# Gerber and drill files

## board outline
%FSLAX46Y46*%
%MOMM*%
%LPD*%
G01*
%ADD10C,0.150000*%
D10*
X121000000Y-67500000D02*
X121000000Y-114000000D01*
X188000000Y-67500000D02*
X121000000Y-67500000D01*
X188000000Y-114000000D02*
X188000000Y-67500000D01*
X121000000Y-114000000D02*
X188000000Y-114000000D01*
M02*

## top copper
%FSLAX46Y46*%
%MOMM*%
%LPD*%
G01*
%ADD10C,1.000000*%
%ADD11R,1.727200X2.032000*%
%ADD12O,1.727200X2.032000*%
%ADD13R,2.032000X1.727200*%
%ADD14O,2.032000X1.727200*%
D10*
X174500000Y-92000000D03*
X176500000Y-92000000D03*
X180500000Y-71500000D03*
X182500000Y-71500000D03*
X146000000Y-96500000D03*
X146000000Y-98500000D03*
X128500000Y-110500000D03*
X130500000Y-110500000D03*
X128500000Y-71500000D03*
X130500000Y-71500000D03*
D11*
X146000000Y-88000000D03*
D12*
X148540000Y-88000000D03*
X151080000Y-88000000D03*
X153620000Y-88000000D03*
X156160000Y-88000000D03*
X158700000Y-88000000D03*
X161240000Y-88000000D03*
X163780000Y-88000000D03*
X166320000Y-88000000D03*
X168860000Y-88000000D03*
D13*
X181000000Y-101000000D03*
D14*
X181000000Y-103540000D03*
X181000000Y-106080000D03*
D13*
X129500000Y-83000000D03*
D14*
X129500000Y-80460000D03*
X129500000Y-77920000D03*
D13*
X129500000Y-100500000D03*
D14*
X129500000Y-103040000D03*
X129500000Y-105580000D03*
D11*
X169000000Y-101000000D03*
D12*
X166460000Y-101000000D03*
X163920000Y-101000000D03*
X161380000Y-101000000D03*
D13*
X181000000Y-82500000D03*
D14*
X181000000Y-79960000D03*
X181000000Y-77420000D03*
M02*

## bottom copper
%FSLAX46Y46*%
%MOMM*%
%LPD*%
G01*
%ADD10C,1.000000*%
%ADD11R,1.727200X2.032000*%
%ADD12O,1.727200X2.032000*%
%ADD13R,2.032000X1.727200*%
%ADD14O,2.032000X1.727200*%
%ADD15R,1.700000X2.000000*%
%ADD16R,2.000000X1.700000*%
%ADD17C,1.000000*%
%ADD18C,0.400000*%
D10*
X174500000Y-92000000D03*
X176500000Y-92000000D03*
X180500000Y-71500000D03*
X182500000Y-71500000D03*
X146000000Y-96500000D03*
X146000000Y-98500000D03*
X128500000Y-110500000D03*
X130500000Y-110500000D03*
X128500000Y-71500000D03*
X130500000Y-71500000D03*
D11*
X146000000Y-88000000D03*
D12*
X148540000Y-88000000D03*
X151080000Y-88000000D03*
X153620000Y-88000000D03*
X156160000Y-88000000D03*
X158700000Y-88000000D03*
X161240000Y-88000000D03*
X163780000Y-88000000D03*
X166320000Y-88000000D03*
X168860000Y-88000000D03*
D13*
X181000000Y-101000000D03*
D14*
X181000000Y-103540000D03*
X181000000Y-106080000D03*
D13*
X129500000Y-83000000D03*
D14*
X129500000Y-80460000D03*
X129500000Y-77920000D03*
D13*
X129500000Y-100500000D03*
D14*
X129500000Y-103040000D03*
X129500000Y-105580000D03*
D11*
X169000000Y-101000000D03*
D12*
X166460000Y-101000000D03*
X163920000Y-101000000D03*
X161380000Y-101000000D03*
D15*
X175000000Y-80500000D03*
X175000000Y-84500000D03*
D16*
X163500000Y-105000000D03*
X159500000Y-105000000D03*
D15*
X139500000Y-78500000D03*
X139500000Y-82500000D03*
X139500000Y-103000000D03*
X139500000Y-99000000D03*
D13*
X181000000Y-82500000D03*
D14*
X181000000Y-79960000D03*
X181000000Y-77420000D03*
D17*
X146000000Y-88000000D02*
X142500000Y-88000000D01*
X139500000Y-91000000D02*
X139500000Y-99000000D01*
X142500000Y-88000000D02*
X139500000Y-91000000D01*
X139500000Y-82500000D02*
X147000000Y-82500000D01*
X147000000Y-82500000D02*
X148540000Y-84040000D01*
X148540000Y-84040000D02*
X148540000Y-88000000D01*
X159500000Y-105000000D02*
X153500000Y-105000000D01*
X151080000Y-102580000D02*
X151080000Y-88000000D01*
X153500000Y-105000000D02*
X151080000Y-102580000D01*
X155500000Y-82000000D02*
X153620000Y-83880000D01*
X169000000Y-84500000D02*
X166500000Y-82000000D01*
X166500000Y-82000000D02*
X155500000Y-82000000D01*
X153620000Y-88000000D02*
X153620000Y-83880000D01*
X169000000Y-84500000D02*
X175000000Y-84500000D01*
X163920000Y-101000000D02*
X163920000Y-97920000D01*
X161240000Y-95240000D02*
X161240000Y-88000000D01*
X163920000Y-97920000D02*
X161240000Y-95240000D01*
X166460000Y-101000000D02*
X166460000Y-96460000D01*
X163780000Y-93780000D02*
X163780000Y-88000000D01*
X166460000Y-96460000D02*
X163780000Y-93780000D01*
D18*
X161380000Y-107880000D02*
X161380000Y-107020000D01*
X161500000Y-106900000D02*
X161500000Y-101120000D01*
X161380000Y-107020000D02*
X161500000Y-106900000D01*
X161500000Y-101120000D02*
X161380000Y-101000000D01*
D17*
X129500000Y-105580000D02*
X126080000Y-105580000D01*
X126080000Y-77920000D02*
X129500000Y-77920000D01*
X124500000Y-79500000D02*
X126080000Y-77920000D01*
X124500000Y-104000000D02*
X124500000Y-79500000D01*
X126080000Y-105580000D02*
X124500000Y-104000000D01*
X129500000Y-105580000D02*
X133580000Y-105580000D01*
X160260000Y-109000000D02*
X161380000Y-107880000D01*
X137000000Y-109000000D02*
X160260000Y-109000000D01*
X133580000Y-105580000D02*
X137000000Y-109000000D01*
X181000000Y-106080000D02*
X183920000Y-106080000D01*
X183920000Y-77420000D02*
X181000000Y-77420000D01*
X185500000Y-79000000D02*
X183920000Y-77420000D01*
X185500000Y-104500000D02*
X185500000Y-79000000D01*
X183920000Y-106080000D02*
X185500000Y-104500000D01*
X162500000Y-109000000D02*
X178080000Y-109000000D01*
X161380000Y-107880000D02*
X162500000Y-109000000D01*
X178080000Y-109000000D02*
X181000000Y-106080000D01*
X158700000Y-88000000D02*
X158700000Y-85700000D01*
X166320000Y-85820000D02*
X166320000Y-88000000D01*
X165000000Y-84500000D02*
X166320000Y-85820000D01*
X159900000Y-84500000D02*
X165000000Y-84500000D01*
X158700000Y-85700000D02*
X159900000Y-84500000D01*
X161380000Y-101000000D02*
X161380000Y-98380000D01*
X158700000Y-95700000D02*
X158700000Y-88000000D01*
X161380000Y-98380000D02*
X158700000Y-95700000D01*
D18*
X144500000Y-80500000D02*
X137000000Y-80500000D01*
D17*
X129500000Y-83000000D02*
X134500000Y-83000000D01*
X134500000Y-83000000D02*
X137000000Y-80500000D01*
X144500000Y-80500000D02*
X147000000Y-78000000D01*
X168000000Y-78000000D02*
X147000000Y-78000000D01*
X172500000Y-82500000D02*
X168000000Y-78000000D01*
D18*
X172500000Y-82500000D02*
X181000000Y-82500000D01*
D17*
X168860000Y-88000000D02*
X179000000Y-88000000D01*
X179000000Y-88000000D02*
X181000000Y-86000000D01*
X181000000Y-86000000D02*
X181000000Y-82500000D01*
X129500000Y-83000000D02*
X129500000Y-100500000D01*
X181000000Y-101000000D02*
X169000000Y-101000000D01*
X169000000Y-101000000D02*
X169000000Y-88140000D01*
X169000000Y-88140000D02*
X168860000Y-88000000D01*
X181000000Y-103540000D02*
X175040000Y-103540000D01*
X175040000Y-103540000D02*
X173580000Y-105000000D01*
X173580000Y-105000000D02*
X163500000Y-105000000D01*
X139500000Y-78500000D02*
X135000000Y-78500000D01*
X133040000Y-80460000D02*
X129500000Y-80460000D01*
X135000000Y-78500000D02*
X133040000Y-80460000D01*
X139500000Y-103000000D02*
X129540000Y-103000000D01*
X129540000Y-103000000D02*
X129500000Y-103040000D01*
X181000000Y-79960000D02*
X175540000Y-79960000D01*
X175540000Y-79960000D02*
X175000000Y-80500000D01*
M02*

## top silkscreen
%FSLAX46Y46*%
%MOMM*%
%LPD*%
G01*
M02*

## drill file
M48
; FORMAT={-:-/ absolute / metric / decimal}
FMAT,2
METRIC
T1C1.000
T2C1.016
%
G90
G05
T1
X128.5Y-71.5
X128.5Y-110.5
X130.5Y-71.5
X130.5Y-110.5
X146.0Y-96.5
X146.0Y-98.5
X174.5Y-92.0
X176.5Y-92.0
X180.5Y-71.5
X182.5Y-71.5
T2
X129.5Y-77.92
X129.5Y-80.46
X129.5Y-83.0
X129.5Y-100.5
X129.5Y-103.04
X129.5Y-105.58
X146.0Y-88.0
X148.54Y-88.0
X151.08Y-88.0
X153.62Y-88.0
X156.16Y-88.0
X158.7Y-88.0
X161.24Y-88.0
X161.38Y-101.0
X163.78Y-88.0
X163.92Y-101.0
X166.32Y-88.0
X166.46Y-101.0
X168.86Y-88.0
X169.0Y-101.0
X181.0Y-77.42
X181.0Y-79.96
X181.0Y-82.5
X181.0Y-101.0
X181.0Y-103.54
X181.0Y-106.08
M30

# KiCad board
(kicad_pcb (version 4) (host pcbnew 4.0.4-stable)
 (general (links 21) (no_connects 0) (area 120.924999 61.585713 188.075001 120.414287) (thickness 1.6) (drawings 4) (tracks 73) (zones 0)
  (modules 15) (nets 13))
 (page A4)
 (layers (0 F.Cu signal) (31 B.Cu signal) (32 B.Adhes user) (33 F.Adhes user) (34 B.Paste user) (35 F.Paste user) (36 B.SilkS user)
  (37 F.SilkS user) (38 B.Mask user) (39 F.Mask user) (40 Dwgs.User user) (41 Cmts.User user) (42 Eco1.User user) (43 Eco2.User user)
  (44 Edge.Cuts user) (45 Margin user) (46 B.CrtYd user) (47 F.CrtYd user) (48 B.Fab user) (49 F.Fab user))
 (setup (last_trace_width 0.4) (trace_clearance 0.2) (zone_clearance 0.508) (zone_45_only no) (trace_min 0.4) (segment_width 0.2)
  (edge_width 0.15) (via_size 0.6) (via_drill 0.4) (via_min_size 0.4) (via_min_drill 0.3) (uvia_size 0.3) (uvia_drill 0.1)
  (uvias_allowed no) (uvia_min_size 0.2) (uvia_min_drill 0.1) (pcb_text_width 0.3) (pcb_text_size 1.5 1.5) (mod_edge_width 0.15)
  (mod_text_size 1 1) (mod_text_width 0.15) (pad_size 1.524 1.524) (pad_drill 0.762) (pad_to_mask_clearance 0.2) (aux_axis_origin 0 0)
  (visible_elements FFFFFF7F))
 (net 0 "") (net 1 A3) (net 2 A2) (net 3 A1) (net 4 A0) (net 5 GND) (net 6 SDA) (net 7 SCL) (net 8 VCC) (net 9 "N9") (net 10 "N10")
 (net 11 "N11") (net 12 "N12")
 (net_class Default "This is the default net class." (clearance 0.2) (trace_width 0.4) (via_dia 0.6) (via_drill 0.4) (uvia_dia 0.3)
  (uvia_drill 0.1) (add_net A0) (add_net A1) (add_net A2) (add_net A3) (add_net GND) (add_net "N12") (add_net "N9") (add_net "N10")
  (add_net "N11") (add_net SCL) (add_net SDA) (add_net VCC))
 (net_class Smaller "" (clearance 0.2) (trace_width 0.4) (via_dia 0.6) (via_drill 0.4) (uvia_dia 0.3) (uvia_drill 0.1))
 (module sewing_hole (layer B.Cu) (at 174 92 270)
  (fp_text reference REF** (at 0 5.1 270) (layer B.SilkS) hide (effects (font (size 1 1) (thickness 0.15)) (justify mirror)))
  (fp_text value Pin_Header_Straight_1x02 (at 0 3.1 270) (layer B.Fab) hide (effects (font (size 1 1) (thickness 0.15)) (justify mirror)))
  (pad 1 thru_hole circle (at 0 -0.5 270) (size 1 1) (drill 1) (layers *.Cu *.Mask))
  (pad 2 thru_hole circle (at 0 -2.5 270) (size 1 1) (drill 1) (layers *.Cu *.Mask)))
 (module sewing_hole (layer B.Cu) (at 180 71.5 270)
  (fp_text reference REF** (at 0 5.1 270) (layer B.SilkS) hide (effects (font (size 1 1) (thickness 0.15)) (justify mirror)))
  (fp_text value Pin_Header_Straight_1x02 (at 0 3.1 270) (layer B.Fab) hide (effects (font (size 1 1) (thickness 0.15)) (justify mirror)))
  (pad 1 thru_hole circle (at 0 -0.5 270) (size 1 1) (drill 1) (layers *.Cu *.Mask))
  (pad 2 thru_hole circle (at 0 -2.5 270) (size 1 1) (drill 1) (layers *.Cu *.Mask)))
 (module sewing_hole (layer B.Cu) (at 146 96 180)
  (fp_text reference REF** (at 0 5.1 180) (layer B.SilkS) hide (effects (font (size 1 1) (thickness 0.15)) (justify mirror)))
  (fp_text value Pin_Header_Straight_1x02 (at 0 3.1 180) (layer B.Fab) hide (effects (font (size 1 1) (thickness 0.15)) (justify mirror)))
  (pad 1 thru_hole circle (at 0 -0.5 180) (size 1 1) (drill 1) (layers *.Cu *.Mask))
  (pad 2 thru_hole circle (at 0 -2.5 180) (size 1 1) (drill 1) (layers *.Cu *.Mask)))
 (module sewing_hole (layer B.Cu) (at 128 110.5 270)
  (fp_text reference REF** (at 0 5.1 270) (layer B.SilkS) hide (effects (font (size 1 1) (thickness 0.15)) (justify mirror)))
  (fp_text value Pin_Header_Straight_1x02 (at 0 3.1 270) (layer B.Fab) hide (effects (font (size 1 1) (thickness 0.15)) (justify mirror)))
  (pad 1 thru_hole circle (at 0 -0.5 270) (size 1 1) (drill 1) (layers *.Cu *.Mask))
  (pad 2 thru_hole circle (at 0 -2.5 270) (size 1 1) (drill 1) (layers *.Cu *.Mask)))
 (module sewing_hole (layer B.Cu) (at 128 71.5 270)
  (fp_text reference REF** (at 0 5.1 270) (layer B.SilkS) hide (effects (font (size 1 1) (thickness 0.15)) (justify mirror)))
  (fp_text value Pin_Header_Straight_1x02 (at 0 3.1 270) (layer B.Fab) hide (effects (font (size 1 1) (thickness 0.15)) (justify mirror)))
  (pad 1 thru_hole circle (at 0 -0.5 270) (size 1 1) (drill 1) (layers *.Cu *.Mask))
  (pad 2 thru_hole circle (at 0 -2.5 270) (size 1 1) (drill 1) (layers *.Cu *.Mask)))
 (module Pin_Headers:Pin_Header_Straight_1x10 (layer B.Cu) (at 146 88 270)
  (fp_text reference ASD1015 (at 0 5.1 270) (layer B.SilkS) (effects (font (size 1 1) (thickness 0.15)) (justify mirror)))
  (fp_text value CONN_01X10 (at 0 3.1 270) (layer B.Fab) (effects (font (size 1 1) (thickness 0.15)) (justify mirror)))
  (pad 1 thru_hole rect (at 0 0 270) (size 2.032 1.7272) (drill 1.016) (layers *.Cu *.Mask) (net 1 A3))
  (pad 2 thru_hole oval (at 0 -2.54 270) (size 2.032 1.7272) (drill 1.016) (layers *.Cu *.Mask) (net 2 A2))
  (pad 3 thru_hole oval (at 0 -5.08 270) (size 2.032 1.7272) (drill 1.016) (layers *.Cu *.Mask) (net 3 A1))
  (pad 4 thru_hole oval (at 0 -7.62 270) (size 2.032 1.7272) (drill 1.016) (layers *.Cu *.Mask) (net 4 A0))
  (pad 5 thru_hole oval (at 0 -10.16 270) (size 2.032 1.7272) (drill 1.016) (layers *.Cu *.Mask))
  (pad 6 thru_hole oval (at 0 -12.7 270) (size 2.032 1.7272) (drill 1.016) (layers *.Cu *.Mask) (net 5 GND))
  (pad 7 thru_hole oval (at 0 -15.24 270) (size 2.032 1.7272) (drill 1.016) (layers *.Cu *.Mask) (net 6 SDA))
  (pad 8 thru_hole oval (at 0 -17.78 270) (size 2.032 1.7272) (drill 1.016) (layers *.Cu *.Mask) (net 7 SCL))
  (pad 9 thru_hole oval (at 0 -20.32 270) (size 2.032 1.7272) (drill 1.016) (layers *.Cu *.Mask) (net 5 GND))
  (pad 10 thru_hole oval (at 0 -22.86 270) (size 2.032 1.7272) (drill 1.016) (layers *.Cu *.Mask) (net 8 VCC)))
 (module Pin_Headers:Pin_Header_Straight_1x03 (layer B.Cu) (at 181 101 180)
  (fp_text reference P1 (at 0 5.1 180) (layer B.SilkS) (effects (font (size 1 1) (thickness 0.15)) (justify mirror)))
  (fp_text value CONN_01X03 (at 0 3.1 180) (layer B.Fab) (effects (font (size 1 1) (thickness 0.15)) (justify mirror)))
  (pad 1 thru_hole rect (at 0 0 180) (size 2.032 1.7272) (drill 1.016) (layers *.Cu *.Mask) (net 8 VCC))
  (pad 2 thru_hole oval (at 0 -2.54 180) (size 2.032 1.7272) (drill 1.016) (layers *.Cu *.Mask) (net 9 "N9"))
  (pad 3 thru_hole oval (at 0 -5.08 180) (size 2.032 1.7272) (drill 1.016) (layers *.Cu *.Mask) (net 5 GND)))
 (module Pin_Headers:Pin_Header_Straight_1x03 (layer B.Cu) (at 129.5 83)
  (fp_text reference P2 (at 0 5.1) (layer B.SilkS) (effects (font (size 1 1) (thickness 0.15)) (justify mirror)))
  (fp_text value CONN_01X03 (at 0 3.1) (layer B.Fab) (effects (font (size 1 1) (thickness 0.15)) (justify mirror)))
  (pad 1 thru_hole rect (at 0 0) (size 2.032 1.7272) (drill 1.016) (layers *.Cu *.Mask) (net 8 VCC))
  (pad 2 thru_hole oval (at 0 -2.54) (size 2.032 1.7272) (drill 1.016) (layers *.Cu *.Mask) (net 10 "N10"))
  (pad 3 thru_hole oval (at 0 -5.08) (size 2.032 1.7272) (drill 1.016) (layers *.Cu *.Mask) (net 5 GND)))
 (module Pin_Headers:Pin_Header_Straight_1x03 (layer B.Cu) (at 129.5 100.5 180)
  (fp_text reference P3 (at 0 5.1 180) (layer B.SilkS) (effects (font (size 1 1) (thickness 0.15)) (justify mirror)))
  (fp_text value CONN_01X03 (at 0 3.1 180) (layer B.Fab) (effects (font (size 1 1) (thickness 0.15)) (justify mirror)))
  (pad 1 thru_hole rect (at 0 0 180) (size 2.032 1.7272) (drill 1.016) (layers *.Cu *.Mask) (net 8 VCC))
  (pad 2 thru_hole oval (at 0 -2.54 180) (size 2.032 1.7272) (drill 1.016) (layers *.Cu *.Mask) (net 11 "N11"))
  (pad 3 thru_hole oval (at 0 -5.08 180) (size 2.032 1.7272) (drill 1.016) (layers *.Cu *.Mask) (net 5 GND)))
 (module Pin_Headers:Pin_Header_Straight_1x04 (layer B.Cu) (at 169 101 90)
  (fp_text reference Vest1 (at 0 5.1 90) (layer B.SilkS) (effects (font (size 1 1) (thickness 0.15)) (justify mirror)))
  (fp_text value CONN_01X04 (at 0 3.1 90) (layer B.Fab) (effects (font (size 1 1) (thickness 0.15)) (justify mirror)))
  (pad 1 thru_hole rect (at 0 0 90) (size 2.032 1.7272) (drill 1.016) (layers *.Cu *.Mask) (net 8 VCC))
  (pad 2 thru_hole oval (at 0 -2.54 90) (size 2.032 1.7272) (drill 1.016) (layers *.Cu *.Mask) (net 7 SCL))
  (pad 3 thru_hole oval (at 0 -5.08 90) (size 2.032 1.7272) (drill 1.016) (layers *.Cu *.Mask) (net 6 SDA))
  (pad 4 thru_hole oval (at 0 -7.62 90) (size 2.032 1.7272) (drill 1.016) (layers *.Cu *.Mask) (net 5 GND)))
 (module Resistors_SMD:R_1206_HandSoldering (layer B.Cu) (at 175 82.5 270)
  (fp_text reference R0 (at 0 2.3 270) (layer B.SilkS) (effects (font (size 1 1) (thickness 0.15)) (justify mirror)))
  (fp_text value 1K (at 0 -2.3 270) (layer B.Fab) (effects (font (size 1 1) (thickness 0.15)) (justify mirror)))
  (pad 1 smd rect (at -2 0 270) (size 2 1.7) (layers B.Cu B.Paste B.Mask) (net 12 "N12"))
  (pad 2 smd rect (at 2 0 270) (size 2 1.7) (layers B.Cu B.Paste B.Mask) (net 4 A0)))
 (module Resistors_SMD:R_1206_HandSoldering (layer B.Cu) (at 161.5 105 180)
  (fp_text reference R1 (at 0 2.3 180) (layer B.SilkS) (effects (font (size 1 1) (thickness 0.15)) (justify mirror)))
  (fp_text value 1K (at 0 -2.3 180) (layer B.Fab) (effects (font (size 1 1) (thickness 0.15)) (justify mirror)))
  (pad 1 smd rect (at -2 0 180) (size 2 1.7) (layers B.Cu B.Paste B.Mask) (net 9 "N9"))
  (pad 2 smd rect (at 2 0 180) (size 2 1.7) (layers B.Cu B.Paste B.Mask) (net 3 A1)))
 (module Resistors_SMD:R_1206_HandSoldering (layer B.Cu) (at 139.5 80.5 270)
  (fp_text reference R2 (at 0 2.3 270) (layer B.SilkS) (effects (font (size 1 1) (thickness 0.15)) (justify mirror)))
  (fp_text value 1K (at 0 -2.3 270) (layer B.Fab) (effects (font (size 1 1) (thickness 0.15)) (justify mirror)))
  (pad 1 smd rect (at -2 0 270) (size 2 1.7) (layers B.Cu B.Paste B.Mask) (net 10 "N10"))
  (pad 2 smd rect (at 2 0 270) (size 2 1.7) (layers B.Cu B.Paste B.Mask) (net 2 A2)))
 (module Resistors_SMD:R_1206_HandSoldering (layer B.Cu) (at 139.5 101 90)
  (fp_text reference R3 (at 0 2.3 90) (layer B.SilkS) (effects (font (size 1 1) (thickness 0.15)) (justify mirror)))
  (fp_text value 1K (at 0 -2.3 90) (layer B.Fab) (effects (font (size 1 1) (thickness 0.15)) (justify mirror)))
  (pad 1 smd rect (at -2 0 90) (size 2 1.7) (layers B.Cu B.Paste B.Mask) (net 11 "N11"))
  (pad 2 smd rect (at 2 0 90) (size 2 1.7) (layers B.Cu B.Paste B.Mask) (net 1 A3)))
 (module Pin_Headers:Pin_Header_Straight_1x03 (layer B.Cu) (at 181 82.5)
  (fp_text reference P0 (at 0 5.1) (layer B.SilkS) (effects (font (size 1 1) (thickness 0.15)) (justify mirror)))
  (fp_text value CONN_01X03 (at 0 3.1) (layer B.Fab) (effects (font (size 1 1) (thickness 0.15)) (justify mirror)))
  (pad 1 thru_hole rect (at 0 0) (size 2.032 1.7272) (drill 1.016) (layers *.Cu *.Mask) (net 8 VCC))
  (pad 2 thru_hole oval (at 0 -2.54) (size 2.032 1.7272) (drill 1.016) (layers *.Cu *.Mask) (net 12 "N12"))
  (pad 3 thru_hole oval (at 0 -5.08) (size 2.032 1.7272) (drill 1.016) (layers *.Cu *.Mask) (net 5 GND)))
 (gr_line (start 121 67.5) (end 121 114) (angle 90) (layer Edge.Cuts) (width 0.15))
 (gr_line (start 188 67.5) (end 121 67.5) (angle 90) (layer Edge.Cuts) (width 0.15))
 (gr_line (start 188 114) (end 188 67.5) (angle 90) (layer Edge.Cuts) (width 0.15))
 (gr_line (start 121 114) (end 188 114) (angle 90) (layer Edge.Cuts) (width 0.15))
 (segment (start 146 88) (end 142.5 88) (width 1) (layer B.Cu) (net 1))
 (segment (start 139.5 91) (end 139.5 99) (width 1) (layer B.Cu) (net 1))
 (segment (start 142.5 88) (end 139.5 91) (width 1) (layer B.Cu) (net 1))
 (segment (start 139.5 82.5) (end 147 82.5) (width 1) (layer B.Cu) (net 2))
 (segment (start 147 82.5) (end 148.54 84.04) (width 1) (layer B.Cu) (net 2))
 (segment (start 148.54 84.04) (end 148.54 88) (width 1) (layer B.Cu) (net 2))
 (segment (start 159.5 105) (end 153.5 105) (width 1) (layer B.Cu) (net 3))
 (segment (start 151.08 102.58) (end 151.08 88) (width 1) (layer B.Cu) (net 3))
 (segment (start 153.5 105) (end 151.08 102.58) (width 1) (layer B.Cu) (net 3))
 (segment (start 155.5 82) (end 153.62 83.88) (width 1) (layer B.Cu) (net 4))
 (segment (start 169 84.5) (end 166.5 82) (width 1) (layer B.Cu) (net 4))
 (segment (start 166.5 82) (end 155.5 82) (width 1) (layer B.Cu) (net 4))
 (segment (start 153.62 88) (end 153.62 83.88) (width 1) (layer B.Cu) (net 4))
 (segment (start 169 84.5) (end 175 84.5) (width 1) (layer B.Cu) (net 4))
 (segment (start 163.92 101) (end 163.92 97.92) (width 1) (layer B.Cu) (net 6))
 (segment (start 161.24 95.24) (end 161.24 88) (width 1) (layer B.Cu) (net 6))
 (segment (start 163.92 97.92) (end 161.24 95.24) (width 1) (layer B.Cu) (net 6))
 (segment (start 166.46 101) (end 166.46 96.46) (width 1) (layer B.Cu) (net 7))
 (segment (start 163.78 93.78) (end 163.78 88) (width 1) (layer B.Cu) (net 7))
 (segment (start 166.46 96.46) (end 163.78 93.78) (width 1) (layer B.Cu) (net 7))
 (segment (start 161.38 107.88) (end 161.38 107.02) (width 0.4) (layer B.Cu) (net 5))
 (segment (start 161.5 106.9) (end 161.5 101.12) (width 0.4) (layer B.Cu) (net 5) (status 800000))
 (segment (start 161.38 107.02) (end 161.5 106.9) (width 0.4) (layer B.Cu) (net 5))
 (segment (start 161.5 101.12) (end 161.38 101) (width 0.4) (layer B.Cu) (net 5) (status C00000))
 (segment (start 129.5 105.58) (end 126.08 105.58) (width 1) (layer B.Cu) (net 5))
 (segment (start 126.08 77.92) (end 129.5 77.92) (width 1) (layer B.Cu) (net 5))
 (segment (start 124.5 79.5) (end 126.08 77.92) (width 1) (layer B.Cu) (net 5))
 (segment (start 124.5 104) (end 124.5 79.5) (width 1) (layer B.Cu) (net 5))
 (segment (start 126.08 105.58) (end 124.5 104) (width 1) (layer B.Cu) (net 5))
 (segment (start 129.5 105.58) (end 133.58 105.58) (width 1) (layer B.Cu) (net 5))
 (segment (start 160.26 109) (end 161.38 107.88) (width 1) (layer B.Cu) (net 5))
 (segment (start 137 109) (end 160.26 109) (width 1) (layer B.Cu) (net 5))
 (segment (start 133.58 105.58) (end 137 109) (width 1) (layer B.Cu) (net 5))
 (segment (start 181 106.08) (end 183.92 106.08) (width 1) (layer B.Cu) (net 5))
 (segment (start 183.92 77.42) (end 181 77.42) (width 1) (layer B.Cu) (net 5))
 (segment (start 185.5 79) (end 183.92 77.42) (width 1) (layer B.Cu) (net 5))
 (segment (start 185.5 104.5) (end 185.5 79) (width 1) (layer B.Cu) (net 5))
 (segment (start 183.92 106.08) (end 185.5 104.5) (width 1) (layer B.Cu) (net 5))
 (segment (start 162.5 109) (end 178.08 109) (width 1) (layer B.Cu) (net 5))
 (segment (start 161.38 107.88) (end 162.5 109) (width 1) (layer B.Cu) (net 5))
 (segment (start 178.08 109) (end 181 106.08) (width 1) (layer B.Cu) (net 5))
 (segment (start 158.7 88) (end 158.7 85.7) (width 1) (layer B.Cu) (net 5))
 (segment (start 166.32 85.82) (end 166.32 88) (width 1) (layer B.Cu) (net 5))
 (segment (start 165 84.5) (end 166.32 85.82) (width 1) (layer B.Cu) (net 5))
 (segment (start 159.9 84.5) (end 165 84.5) (width 1) (layer B.Cu) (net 5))
 (segment (start 158.7 85.7) (end 159.9 84.5) (width 1) (layer B.Cu) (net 5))
 (segment (start 161.38 101) (end 161.38 98.38) (width 1) (layer B.Cu) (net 5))
 (segment (start 158.7 95.7) (end 158.7 88) (width 1) (layer B.Cu) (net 5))
 (segment (start 161.38 98.38) (end 158.7 95.7) (width 1) (layer B.Cu) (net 5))
 (segment (start 144.5 80.5) (end 137 80.5) (width 0.4) (layer B.Cu) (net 8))
 (segment (start 129.5 83) (end 134.5 83) (width 1) (layer B.Cu) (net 8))
 (segment (start 134.5 83) (end 137 80.5) (width 1) (layer B.Cu) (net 8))
 (segment (start 144.5 80.5) (end 147 78) (width 1) (layer B.Cu) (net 8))
 (segment (start 168 78) (end 147 78) (width 1) (layer B.Cu) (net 8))
 (segment (start 172.5 82.5) (end 168 78) (width 1) (layer B.Cu) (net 8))
 (segment (start 172.5 82.5) (end 181 82.5) (width 0.4) (layer B.Cu) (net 8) (status 800000))
 (segment (start 168.86 88) (end 179 88) (width 1) (layer B.Cu) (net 8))
 (segment (start 179 88) (end 181 86) (width 1) (layer B.Cu) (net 8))
 (segment (start 181 86) (end 181 82.5) (width 1) (layer B.Cu) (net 8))
 (segment (start 129.5 83) (end 129.5 100.5) (width 1) (layer B.Cu) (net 8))
 (segment (start 181 101) (end 169 101) (width 1) (layer B.Cu) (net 8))
 (segment (start 169 101) (end 169 88.14) (width 1) (layer B.Cu) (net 8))
 (segment (start 169 88.14) (end 168.86 88) (width 1) (layer B.Cu) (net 8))
 (segment (start 181 103.54) (end 175.04 103.54) (width 1) (layer B.Cu) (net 9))
 (segment (start 175.04 103.54) (end 173.58 105) (width 1) (layer B.Cu) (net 9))
 (segment (start 173.58 105) (end 163.5 105) (width 1) (layer B.Cu) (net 9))
 (segment (start 139.5 78.5) (end 135 78.5) (width 1) (layer B.Cu) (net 10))
 (segment (start 133.04 80.46) (end 129.5 80.46) (width 1) (layer B.Cu) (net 10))
 (segment (start 135 78.5) (end 133.04 80.46) (width 1) (layer B.Cu) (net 10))
 (segment (start 139.5 103) (end 129.54 103) (width 1) (layer B.Cu) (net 11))
 (segment (start 129.54 103) (end 129.5 103.04) (width 1) (layer B.Cu) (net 11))
 (segment (start 181 79.96) (end 175.54 79.96) (width 1) (layer B.Cu) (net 12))
 (segment (start 175.54 79.96) (end 175 80.5) (width 1) (layer B.Cu) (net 12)))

